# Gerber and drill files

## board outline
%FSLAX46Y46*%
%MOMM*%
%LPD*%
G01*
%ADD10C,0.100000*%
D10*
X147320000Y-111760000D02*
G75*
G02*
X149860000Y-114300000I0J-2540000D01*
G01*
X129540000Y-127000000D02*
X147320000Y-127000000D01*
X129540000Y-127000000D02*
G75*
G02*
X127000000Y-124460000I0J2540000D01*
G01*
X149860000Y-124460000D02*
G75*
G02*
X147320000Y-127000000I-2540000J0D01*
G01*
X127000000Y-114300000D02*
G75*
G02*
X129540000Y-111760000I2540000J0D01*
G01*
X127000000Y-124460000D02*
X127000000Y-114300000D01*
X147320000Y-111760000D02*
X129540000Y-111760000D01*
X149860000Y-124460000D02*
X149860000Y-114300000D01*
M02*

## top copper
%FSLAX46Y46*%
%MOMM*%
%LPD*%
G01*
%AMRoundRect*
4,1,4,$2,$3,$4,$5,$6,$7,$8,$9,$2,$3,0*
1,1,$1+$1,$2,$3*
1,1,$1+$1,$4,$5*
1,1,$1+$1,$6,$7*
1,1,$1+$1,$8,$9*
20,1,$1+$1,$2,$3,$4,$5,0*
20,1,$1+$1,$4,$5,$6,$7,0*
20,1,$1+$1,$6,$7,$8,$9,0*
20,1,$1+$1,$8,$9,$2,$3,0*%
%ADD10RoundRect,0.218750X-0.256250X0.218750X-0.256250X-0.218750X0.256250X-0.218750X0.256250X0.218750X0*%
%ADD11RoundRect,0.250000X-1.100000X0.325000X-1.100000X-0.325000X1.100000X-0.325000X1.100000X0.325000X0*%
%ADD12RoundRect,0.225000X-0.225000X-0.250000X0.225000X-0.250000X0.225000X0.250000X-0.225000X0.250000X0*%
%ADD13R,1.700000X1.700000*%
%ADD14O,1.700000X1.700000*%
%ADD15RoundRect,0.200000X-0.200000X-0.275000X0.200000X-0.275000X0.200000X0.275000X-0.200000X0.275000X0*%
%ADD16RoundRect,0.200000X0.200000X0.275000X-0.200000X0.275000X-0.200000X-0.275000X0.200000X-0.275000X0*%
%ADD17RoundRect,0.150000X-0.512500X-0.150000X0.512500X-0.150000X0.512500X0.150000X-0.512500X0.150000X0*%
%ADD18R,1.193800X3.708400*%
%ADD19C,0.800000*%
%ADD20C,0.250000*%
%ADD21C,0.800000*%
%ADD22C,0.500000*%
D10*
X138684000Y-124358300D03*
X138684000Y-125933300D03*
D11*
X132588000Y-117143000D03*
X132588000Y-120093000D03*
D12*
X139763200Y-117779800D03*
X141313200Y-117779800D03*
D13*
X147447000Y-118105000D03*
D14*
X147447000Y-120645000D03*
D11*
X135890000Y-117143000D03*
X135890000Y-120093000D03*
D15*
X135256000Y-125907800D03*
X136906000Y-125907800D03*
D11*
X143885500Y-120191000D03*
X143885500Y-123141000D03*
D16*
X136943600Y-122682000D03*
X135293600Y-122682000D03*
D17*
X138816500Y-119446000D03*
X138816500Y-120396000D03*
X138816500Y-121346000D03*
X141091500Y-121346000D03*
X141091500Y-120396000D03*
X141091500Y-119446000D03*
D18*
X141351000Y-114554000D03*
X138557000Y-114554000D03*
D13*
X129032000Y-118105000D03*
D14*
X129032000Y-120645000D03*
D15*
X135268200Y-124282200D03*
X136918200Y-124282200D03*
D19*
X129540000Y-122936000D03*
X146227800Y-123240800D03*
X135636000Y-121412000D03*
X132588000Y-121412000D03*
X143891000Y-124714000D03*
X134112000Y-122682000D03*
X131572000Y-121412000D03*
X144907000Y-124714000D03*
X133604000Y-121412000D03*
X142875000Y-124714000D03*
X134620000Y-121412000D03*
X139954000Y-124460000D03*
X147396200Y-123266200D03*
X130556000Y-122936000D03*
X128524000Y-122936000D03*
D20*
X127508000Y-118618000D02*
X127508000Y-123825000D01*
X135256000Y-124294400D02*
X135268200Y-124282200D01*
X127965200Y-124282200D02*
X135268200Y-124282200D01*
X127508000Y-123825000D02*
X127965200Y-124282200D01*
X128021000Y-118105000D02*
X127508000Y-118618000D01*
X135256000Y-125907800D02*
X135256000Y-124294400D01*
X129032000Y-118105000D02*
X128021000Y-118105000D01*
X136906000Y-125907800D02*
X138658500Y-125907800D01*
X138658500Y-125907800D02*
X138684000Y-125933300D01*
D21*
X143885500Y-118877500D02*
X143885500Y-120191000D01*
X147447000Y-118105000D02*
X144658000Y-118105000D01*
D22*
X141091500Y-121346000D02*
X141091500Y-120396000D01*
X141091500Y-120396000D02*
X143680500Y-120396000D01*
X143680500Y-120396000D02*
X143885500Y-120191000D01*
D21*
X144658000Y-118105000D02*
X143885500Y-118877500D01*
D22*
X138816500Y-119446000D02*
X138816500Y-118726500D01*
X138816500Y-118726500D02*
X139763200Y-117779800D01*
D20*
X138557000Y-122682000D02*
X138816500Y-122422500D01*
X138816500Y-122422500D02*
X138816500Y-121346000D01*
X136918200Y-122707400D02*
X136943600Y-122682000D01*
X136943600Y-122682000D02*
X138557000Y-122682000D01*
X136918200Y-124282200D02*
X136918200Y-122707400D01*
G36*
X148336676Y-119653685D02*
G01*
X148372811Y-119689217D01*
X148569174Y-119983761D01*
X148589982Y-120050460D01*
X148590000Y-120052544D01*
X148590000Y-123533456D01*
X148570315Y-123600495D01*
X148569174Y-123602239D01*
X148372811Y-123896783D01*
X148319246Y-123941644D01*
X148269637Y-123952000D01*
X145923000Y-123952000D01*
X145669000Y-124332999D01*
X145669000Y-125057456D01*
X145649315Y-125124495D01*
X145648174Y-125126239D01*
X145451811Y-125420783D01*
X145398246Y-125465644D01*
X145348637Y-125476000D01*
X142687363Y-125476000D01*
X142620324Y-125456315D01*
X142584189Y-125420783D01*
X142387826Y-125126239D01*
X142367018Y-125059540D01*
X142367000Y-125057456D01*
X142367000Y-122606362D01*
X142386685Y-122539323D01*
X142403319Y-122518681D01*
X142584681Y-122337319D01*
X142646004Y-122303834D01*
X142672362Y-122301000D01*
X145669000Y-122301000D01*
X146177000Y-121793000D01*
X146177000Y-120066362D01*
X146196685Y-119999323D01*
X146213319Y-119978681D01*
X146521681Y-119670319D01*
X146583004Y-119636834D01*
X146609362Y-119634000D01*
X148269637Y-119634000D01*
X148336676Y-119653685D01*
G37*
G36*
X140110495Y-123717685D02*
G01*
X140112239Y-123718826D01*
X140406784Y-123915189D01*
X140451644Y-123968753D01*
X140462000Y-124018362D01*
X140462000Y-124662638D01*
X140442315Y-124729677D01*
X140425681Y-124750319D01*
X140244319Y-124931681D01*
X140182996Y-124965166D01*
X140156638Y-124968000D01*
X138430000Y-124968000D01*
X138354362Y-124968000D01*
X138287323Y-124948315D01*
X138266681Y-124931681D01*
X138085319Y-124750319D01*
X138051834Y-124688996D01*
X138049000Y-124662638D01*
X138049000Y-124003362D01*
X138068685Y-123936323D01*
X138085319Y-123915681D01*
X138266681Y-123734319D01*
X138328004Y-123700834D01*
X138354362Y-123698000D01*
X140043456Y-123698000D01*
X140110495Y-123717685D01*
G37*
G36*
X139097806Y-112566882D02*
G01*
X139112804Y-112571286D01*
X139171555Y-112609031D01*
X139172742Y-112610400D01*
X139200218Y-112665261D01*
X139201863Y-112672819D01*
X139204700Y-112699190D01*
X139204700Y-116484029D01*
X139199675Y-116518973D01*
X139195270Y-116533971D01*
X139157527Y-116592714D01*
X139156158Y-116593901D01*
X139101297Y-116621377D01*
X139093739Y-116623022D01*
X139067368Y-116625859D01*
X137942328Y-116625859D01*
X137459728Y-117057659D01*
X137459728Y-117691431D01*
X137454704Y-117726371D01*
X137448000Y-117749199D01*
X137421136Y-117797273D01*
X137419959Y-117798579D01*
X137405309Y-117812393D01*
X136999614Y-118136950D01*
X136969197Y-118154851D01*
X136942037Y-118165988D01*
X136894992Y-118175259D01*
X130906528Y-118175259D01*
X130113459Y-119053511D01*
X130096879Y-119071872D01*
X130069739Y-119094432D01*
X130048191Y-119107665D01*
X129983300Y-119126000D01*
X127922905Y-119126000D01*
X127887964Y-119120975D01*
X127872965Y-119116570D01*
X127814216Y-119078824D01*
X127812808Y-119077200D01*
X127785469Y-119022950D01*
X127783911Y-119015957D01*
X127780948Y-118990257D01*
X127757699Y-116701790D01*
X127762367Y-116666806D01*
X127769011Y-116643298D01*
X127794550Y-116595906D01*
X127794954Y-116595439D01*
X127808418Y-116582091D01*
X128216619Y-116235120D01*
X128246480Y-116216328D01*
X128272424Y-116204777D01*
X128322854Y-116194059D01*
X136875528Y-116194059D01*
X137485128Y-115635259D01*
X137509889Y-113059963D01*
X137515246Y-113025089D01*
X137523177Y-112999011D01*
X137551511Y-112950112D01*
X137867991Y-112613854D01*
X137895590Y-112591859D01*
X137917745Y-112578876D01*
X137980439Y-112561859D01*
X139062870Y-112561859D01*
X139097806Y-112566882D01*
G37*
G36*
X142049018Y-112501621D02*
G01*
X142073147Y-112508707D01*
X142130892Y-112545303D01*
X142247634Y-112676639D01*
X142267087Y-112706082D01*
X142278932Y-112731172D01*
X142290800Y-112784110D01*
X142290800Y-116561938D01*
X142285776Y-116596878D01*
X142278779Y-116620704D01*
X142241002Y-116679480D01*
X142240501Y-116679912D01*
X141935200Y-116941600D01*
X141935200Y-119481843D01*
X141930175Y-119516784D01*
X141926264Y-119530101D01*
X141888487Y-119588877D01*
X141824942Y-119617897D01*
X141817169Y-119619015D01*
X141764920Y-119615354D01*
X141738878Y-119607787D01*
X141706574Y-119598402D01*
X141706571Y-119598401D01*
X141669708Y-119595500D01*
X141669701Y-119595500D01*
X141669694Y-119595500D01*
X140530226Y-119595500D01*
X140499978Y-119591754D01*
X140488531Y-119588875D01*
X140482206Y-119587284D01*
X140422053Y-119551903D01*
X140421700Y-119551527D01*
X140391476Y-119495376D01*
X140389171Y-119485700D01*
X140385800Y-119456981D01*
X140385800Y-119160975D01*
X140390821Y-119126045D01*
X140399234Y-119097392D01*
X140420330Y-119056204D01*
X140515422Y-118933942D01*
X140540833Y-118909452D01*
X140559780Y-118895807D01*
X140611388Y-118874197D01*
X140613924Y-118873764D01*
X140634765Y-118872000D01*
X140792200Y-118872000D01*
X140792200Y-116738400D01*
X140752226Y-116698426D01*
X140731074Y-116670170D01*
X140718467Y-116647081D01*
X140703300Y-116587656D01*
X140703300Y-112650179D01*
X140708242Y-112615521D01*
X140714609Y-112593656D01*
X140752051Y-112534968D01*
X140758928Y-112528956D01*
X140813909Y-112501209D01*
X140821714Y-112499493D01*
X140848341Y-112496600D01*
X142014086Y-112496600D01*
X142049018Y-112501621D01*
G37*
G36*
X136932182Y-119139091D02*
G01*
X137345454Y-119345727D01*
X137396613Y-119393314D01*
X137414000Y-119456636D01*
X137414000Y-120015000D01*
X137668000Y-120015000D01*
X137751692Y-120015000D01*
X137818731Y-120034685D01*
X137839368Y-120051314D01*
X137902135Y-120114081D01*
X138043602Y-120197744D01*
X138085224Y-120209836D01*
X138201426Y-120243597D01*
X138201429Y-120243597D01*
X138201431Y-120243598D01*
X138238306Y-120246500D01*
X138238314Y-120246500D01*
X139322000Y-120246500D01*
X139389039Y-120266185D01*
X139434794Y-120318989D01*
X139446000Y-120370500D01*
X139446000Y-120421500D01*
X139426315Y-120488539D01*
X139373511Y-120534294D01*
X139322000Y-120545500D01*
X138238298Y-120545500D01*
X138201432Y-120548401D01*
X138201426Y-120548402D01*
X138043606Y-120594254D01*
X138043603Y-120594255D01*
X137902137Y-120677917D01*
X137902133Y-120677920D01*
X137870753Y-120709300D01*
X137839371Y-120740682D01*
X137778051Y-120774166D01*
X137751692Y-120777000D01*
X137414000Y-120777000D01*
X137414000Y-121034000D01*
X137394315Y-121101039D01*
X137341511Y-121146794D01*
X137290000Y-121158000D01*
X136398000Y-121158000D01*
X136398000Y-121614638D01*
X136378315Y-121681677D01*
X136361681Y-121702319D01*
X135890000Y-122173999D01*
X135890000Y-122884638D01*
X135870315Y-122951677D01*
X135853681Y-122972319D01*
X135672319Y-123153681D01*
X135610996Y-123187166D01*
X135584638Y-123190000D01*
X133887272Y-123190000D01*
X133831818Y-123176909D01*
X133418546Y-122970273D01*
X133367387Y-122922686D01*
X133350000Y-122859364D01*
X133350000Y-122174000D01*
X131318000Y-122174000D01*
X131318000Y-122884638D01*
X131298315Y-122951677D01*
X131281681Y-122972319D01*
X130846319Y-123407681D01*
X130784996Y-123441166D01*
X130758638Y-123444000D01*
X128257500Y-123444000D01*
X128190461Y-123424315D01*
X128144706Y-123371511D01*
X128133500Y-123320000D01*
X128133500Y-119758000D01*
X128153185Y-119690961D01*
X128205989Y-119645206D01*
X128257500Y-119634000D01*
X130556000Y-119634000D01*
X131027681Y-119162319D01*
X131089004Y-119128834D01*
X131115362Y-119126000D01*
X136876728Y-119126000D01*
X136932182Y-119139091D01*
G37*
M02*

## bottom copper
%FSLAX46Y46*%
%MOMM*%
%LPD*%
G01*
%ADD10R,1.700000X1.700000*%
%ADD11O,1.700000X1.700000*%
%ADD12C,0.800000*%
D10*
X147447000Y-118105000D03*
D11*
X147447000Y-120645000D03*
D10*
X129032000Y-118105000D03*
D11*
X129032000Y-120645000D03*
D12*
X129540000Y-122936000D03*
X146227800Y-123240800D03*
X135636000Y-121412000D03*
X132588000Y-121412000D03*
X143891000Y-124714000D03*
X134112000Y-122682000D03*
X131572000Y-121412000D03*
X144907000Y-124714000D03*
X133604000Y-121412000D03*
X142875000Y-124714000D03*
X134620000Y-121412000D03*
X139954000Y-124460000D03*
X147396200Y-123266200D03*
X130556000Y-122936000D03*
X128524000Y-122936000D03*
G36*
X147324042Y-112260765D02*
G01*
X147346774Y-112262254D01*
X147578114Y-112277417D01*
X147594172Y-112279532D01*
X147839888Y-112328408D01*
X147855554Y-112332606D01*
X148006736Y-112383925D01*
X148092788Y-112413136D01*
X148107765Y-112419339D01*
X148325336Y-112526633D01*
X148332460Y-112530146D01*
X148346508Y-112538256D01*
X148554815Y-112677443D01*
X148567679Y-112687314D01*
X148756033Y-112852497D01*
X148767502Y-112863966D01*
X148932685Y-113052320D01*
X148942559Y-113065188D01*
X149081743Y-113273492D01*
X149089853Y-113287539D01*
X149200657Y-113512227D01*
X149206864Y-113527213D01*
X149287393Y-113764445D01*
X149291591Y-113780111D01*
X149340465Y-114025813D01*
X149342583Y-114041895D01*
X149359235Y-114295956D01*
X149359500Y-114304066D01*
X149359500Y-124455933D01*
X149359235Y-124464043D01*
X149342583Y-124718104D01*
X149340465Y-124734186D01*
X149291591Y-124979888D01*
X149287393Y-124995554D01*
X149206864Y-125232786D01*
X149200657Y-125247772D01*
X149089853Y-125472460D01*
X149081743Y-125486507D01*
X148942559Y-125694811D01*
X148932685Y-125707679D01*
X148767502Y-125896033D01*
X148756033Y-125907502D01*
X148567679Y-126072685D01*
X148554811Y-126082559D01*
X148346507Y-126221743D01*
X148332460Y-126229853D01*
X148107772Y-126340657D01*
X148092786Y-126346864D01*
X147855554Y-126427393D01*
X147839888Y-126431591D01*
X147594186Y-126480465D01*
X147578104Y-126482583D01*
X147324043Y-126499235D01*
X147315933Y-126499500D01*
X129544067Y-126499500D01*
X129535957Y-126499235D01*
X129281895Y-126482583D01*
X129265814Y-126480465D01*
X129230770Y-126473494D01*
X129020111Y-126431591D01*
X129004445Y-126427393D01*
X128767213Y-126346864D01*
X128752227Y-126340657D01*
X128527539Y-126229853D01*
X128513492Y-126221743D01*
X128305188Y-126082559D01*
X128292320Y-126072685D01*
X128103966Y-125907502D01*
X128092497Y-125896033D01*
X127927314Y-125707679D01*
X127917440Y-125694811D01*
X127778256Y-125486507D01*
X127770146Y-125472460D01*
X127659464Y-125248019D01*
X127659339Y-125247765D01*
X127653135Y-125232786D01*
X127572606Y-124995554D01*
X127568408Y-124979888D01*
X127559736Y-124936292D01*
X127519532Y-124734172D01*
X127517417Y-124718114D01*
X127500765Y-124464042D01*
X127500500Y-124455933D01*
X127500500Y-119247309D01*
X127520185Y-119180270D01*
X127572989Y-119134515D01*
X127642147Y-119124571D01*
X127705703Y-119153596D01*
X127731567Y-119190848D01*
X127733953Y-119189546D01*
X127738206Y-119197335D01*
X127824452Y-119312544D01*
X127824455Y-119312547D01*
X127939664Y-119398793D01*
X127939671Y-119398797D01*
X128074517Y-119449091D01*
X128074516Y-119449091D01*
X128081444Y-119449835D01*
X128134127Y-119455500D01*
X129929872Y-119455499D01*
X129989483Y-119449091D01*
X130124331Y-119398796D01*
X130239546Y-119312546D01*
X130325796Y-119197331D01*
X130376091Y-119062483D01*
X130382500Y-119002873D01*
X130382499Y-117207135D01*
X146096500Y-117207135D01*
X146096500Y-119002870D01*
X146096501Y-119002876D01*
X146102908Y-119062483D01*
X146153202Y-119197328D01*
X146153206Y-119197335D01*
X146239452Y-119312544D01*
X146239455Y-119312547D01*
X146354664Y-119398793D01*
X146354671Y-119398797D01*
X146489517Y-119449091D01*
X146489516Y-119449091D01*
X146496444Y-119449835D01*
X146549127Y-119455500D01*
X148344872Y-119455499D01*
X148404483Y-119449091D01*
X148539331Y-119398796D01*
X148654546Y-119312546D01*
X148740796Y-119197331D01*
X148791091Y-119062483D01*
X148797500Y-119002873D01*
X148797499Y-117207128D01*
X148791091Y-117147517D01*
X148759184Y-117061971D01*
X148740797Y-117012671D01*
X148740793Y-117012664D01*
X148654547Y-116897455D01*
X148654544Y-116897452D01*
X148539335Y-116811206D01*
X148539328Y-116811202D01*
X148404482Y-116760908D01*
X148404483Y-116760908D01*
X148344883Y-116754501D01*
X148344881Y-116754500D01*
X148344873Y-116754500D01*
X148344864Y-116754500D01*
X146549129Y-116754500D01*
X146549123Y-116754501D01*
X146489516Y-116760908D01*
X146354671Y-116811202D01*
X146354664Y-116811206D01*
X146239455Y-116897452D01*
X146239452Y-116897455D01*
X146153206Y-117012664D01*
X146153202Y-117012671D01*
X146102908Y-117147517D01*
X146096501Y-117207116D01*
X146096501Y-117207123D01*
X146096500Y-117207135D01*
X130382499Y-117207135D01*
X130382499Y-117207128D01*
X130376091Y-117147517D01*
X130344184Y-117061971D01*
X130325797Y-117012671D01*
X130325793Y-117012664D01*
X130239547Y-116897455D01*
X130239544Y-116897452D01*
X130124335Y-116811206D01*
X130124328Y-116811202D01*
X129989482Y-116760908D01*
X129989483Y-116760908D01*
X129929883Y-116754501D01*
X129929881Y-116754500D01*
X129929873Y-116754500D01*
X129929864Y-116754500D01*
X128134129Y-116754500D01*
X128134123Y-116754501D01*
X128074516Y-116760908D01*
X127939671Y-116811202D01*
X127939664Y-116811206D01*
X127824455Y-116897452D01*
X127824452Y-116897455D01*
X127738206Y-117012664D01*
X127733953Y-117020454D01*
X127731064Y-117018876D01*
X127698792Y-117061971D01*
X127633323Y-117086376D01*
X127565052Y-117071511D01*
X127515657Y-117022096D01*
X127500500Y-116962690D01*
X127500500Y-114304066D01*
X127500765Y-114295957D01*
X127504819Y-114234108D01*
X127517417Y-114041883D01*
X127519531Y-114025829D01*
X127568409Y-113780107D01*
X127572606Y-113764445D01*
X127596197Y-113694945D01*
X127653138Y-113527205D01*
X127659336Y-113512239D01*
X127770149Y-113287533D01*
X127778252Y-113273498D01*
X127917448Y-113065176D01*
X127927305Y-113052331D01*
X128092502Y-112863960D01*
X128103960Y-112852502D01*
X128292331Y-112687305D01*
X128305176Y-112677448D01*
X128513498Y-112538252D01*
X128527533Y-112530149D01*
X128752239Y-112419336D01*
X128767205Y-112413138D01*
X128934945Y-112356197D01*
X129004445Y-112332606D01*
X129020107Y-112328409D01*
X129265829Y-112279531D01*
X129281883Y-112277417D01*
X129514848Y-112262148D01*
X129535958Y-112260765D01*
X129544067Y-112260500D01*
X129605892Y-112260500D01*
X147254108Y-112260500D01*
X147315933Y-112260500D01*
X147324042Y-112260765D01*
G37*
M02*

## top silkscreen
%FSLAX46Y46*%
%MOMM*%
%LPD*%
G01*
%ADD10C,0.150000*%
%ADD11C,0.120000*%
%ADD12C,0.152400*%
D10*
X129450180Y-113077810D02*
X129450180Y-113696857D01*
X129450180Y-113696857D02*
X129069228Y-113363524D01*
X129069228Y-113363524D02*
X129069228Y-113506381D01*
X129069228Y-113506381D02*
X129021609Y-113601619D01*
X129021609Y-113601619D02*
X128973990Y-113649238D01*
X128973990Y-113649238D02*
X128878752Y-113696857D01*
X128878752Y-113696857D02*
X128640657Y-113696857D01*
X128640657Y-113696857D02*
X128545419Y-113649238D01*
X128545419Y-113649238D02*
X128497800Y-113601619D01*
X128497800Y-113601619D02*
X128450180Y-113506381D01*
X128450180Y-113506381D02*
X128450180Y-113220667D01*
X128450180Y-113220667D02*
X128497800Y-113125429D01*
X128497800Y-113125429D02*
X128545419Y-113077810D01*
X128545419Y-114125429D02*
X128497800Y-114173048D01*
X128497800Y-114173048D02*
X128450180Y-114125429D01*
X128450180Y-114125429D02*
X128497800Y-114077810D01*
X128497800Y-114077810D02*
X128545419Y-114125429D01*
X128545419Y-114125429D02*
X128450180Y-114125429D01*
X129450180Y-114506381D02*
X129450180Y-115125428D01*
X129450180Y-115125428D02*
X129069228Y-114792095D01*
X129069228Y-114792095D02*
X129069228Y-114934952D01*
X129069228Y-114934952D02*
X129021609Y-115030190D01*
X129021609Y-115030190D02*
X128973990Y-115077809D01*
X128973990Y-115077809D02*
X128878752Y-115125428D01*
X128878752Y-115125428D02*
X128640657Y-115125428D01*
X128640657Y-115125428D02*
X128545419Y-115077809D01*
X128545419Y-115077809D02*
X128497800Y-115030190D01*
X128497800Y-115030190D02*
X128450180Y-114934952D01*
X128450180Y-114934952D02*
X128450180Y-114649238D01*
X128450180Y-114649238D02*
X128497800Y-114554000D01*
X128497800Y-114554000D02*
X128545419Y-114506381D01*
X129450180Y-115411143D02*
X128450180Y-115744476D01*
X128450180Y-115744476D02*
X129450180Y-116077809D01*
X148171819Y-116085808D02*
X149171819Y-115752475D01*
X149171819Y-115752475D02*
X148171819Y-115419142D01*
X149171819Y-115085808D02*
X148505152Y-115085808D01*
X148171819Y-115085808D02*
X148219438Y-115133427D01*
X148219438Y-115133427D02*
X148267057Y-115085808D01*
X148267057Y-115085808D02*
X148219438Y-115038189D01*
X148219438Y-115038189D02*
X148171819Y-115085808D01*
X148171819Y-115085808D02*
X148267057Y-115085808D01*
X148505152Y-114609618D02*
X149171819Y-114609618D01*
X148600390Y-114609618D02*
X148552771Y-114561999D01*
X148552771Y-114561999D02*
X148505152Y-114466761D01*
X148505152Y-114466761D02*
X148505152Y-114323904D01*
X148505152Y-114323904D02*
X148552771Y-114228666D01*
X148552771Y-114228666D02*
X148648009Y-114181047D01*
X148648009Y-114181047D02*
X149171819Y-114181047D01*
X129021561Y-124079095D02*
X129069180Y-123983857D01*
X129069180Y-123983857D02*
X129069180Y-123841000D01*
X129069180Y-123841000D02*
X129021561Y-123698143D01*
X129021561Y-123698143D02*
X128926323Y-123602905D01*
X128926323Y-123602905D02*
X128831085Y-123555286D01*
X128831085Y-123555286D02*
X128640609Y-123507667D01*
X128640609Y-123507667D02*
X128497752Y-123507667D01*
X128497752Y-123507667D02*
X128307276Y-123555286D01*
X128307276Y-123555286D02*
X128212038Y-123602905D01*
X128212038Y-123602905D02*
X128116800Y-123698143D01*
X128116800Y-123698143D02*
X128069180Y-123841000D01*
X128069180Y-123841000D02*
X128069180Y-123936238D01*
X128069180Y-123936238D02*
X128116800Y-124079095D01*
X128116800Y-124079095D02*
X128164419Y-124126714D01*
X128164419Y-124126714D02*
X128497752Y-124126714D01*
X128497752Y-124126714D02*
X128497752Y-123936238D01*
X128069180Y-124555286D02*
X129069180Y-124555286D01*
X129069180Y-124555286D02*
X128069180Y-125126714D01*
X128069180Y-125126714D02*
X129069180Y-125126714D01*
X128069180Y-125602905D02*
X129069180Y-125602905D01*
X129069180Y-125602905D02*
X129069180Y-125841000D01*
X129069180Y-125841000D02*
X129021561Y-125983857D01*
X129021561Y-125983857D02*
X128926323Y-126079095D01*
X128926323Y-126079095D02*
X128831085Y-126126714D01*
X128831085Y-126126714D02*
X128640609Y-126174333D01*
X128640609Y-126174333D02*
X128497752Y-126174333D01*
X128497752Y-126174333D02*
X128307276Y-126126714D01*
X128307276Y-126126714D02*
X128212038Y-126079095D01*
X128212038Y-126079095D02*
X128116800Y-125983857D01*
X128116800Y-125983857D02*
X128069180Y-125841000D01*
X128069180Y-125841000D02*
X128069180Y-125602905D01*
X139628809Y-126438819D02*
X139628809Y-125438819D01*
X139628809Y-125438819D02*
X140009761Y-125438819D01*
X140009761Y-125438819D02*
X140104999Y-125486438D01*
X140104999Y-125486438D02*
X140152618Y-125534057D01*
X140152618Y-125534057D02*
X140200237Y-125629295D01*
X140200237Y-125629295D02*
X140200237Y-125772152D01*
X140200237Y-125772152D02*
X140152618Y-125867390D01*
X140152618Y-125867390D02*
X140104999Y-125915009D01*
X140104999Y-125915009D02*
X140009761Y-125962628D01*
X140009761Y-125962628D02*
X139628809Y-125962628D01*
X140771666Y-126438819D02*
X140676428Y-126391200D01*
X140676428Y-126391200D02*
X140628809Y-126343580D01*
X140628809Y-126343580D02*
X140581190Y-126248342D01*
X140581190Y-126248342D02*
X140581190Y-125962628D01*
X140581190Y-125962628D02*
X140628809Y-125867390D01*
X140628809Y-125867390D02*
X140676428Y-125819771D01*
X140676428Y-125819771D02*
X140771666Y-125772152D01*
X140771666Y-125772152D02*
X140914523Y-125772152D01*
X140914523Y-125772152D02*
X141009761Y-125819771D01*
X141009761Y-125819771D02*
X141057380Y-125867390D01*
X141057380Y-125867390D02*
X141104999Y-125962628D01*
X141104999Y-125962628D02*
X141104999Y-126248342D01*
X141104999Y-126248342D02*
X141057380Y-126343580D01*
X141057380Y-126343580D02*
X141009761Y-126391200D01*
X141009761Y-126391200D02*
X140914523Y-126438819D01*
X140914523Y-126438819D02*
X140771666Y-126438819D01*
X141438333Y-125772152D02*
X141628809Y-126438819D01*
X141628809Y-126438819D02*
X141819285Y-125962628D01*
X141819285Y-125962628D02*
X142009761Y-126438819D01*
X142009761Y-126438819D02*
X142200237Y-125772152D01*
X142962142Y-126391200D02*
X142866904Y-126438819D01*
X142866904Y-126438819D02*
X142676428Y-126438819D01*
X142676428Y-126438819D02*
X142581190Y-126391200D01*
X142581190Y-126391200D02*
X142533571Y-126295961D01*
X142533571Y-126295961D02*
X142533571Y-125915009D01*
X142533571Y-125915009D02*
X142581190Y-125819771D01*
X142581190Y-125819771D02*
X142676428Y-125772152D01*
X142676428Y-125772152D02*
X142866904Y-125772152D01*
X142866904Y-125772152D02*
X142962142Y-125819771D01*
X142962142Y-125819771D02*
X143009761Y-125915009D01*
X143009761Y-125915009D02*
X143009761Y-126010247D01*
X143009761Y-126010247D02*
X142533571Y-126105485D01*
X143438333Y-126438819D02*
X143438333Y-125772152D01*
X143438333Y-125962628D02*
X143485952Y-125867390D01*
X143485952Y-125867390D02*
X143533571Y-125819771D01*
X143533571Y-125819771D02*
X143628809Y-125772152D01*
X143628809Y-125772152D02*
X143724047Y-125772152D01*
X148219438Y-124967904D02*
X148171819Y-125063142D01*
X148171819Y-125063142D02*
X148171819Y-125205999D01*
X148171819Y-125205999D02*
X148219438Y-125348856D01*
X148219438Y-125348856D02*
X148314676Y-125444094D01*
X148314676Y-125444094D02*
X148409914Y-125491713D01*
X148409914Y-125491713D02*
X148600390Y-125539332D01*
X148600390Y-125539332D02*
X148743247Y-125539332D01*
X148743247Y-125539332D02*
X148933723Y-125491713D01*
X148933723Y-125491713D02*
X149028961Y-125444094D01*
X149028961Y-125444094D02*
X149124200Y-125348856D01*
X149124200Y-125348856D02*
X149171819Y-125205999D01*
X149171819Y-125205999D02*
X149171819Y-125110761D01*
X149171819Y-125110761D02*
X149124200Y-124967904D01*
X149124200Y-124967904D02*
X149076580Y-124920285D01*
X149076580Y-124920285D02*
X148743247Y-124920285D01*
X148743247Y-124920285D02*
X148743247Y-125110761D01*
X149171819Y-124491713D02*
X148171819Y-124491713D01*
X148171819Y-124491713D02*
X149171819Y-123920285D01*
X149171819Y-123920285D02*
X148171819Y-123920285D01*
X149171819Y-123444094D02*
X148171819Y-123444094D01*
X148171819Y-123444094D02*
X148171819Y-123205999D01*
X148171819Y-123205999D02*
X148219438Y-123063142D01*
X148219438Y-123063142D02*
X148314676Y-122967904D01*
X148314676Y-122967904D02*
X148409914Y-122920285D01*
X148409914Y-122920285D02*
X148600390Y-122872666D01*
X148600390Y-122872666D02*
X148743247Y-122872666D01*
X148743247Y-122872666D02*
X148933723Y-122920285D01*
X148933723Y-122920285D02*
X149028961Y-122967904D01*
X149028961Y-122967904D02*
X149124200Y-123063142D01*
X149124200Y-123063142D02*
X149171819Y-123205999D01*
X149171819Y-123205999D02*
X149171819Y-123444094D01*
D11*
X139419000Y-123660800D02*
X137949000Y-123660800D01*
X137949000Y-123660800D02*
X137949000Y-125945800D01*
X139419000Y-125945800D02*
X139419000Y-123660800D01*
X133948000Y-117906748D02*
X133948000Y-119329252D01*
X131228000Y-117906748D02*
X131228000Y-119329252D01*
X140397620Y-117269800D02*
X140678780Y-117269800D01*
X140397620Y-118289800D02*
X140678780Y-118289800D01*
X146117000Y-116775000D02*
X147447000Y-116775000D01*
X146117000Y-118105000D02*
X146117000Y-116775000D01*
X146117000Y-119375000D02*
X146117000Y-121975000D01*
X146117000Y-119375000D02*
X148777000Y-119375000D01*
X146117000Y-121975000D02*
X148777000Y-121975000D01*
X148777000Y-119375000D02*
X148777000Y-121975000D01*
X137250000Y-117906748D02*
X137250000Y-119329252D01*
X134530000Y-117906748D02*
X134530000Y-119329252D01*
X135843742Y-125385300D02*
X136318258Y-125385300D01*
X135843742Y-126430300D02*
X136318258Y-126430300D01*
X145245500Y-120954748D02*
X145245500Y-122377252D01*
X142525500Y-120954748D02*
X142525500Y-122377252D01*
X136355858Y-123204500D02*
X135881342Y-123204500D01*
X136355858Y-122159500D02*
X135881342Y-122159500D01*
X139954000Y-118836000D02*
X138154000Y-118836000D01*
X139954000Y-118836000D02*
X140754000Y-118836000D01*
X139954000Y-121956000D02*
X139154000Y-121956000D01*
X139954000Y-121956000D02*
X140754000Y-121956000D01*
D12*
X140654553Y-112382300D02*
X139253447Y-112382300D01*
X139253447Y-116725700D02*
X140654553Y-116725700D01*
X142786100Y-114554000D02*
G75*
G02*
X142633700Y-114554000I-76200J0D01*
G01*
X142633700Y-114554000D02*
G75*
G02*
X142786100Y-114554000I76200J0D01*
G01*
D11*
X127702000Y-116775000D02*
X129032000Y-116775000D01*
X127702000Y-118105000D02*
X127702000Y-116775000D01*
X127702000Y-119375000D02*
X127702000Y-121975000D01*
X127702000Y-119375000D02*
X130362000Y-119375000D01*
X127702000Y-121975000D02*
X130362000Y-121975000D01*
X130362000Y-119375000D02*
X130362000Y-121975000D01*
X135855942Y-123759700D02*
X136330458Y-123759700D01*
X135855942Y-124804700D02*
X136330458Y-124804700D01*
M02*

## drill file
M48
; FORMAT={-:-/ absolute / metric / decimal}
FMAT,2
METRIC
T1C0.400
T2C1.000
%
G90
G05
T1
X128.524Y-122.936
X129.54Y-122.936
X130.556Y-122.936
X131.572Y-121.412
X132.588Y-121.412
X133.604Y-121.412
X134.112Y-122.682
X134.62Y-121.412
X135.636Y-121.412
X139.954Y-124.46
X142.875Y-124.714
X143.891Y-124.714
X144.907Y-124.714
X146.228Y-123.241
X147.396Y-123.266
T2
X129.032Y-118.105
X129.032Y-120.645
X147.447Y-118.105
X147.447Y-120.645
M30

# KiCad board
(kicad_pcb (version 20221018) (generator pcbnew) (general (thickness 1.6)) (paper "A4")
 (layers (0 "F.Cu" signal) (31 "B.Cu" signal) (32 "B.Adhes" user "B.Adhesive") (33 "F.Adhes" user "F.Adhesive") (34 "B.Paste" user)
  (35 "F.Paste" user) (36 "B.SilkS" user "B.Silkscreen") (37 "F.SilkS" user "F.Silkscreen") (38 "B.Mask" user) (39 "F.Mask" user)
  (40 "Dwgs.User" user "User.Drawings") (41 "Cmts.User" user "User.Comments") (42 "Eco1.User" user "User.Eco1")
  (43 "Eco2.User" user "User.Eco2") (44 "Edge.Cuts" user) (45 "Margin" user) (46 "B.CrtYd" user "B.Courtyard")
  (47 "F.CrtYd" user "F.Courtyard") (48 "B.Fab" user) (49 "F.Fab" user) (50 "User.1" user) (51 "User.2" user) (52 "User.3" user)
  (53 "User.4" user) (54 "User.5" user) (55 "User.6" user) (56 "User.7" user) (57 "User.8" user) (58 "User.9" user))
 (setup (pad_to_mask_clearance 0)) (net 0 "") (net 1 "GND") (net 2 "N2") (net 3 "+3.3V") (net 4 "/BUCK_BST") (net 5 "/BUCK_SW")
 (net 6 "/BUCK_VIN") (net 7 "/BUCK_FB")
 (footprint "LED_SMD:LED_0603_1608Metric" (layer "F.Cu") (at 138.684 125.1458 -90)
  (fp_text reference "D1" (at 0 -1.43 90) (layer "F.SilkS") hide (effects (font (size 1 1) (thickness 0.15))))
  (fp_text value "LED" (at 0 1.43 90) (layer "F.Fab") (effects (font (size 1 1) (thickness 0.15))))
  (fp_line (start -1.485 -0.735) (end -1.485 0.735) (stroke (width 0.12) (type solid)) (layer "F.SilkS"))
  (fp_line (start -1.485 0.735) (end 0.8 0.735) (stroke (width 0.12) (type solid)) (layer "F.SilkS"))
  (fp_line (start 0.8 -0.735) (end -1.485 -0.735) (stroke (width 0.12) (type solid)) (layer "F.SilkS"))
  (pad "1" smd roundrect (at -0.7875 0 270) (size 0.875 0.95) (layers "F.Cu" "F.Paste" "F.Mask") (roundrect_rratio 0.25) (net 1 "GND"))
  (pad "2" smd roundrect (at 0.7875 0 270) (size 0.875 0.95) (layers "F.Cu" "F.Paste" "F.Mask") (roundrect_rratio 0.25) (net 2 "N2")))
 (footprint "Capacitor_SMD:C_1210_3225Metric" (layer "F.Cu") (at 132.588 118.618 -90)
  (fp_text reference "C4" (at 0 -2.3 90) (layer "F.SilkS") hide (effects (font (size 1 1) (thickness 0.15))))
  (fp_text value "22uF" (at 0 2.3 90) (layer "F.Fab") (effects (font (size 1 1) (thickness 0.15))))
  (fp_line (start -0.711252 -1.36) (end 0.711252 -1.36) (stroke (width 0.12) (type solid)) (layer "F.SilkS"))
  (fp_line (start -0.711252 1.36) (end 0.711252 1.36) (stroke (width 0.12) (type solid)) (layer "F.SilkS"))
  (pad "1" smd roundrect (at -1.475 0 270) (size 1.15 2.7) (layers "F.Cu" "F.Paste" "F.Mask") (roundrect_rratio 0.217391) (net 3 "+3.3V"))
  (pad "2" smd roundrect (at 1.475 0 270) (size 1.15 2.7) (layers "F.Cu" "F.Paste" "F.Mask") (roundrect_rratio 0.217391) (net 1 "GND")))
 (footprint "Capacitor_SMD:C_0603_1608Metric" (layer "F.Cu") (at 140.5382 117.7798)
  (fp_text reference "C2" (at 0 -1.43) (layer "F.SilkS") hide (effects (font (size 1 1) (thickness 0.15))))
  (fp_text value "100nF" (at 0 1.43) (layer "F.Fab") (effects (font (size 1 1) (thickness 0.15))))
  (fp_line (start -0.14058 -0.51) (end 0.14058 -0.51) (stroke (width 0.12) (type solid)) (layer "F.SilkS"))
  (fp_line (start -0.14058 0.51) (end 0.14058 0.51) (stroke (width 0.12) (type solid)) (layer "F.SilkS"))
  (pad "1" smd roundrect (at -0.775 0) (size 0.9 0.95) (layers "F.Cu" "F.Paste" "F.Mask") (roundrect_rratio 0.25) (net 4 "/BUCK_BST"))
  (pad "2" smd roundrect (at 0.775 0) (size 0.9 0.95) (layers "F.Cu" "F.Paste" "F.Mask") (roundrect_rratio 0.25) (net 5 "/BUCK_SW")))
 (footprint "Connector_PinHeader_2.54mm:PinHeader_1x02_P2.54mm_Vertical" (layer "F.Cu") (at 147.447 118.105)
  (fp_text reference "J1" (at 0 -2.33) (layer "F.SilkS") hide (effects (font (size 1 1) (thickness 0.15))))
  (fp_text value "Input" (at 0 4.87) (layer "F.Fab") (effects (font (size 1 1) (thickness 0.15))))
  (fp_line (start -1.33 -1.33) (end 0 -1.33) (stroke (width 0.12) (type solid)) (layer "F.SilkS"))
  (fp_line (start -1.33 0) (end -1.33 -1.33) (stroke (width 0.12) (type solid)) (layer "F.SilkS"))
  (fp_line (start -1.33 1.27) (end -1.33 3.87) (stroke (width 0.12) (type solid)) (layer "F.SilkS"))
  (fp_line (start -1.33 1.27) (end 1.33 1.27) (stroke (width 0.12) (type solid)) (layer "F.SilkS"))
  (fp_line (start -1.33 3.87) (end 1.33 3.87) (stroke (width 0.12) (type solid)) (layer "F.SilkS"))
  (fp_line (start 1.33 1.27) (end 1.33 3.87) (stroke (width 0.12) (type solid)) (layer "F.SilkS"))
  (pad "1" thru_hole rect (at 0 0) (size 1.7 1.7) (drill 1) (layers "*.Cu" "*.Mask") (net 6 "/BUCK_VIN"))
  (pad "2" thru_hole oval (at 0 2.54) (size 1.7 1.7) (drill 1) (layers "*.Cu" "*.Mask") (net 1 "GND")))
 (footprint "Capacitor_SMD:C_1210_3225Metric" (layer "F.Cu") (at 135.89 118.618 -90)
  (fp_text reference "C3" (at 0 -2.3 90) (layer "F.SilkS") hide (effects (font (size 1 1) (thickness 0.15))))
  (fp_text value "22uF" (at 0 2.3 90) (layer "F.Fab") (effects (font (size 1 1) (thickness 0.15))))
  (fp_line (start -0.711252 -1.36) (end 0.711252 -1.36) (stroke (width 0.12) (type solid)) (layer "F.SilkS"))
  (fp_line (start -0.711252 1.36) (end 0.711252 1.36) (stroke (width 0.12) (type solid)) (layer "F.SilkS"))
  (pad "1" smd roundrect (at -1.475 0 270) (size 1.15 2.7) (layers "F.Cu" "F.Paste" "F.Mask") (roundrect_rratio 0.217391) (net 3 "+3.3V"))
  (pad "2" smd roundrect (at 1.475 0 270) (size 1.15 2.7) (layers "F.Cu" "F.Paste" "F.Mask") (roundrect_rratio 0.217391) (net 1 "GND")))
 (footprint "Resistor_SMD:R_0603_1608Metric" (layer "F.Cu") (at 136.081 125.9078)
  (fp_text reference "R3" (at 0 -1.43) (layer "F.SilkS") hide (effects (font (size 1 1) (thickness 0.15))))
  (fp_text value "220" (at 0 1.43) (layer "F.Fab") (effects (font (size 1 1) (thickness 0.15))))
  (fp_line (start -0.237258 -0.5225) (end 0.237258 -0.5225) (stroke (width 0.12) (type solid)) (layer "F.SilkS"))
  (fp_line (start -0.237258 0.5225) (end 0.237258 0.5225) (stroke (width 0.12) (type solid)) (layer "F.SilkS"))
  (pad "1" smd roundrect (at -0.825 0) (size 0.8 0.95) (layers "F.Cu" "F.Paste" "F.Mask") (roundrect_rratio 0.25) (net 3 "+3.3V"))
  (pad "2" smd roundrect (at 0.825 0) (size 0.8 0.95) (layers "F.Cu" "F.Paste" "F.Mask") (roundrect_rratio 0.25) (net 2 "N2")))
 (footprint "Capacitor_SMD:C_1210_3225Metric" (layer "F.Cu") (at 143.8855 121.666 -90)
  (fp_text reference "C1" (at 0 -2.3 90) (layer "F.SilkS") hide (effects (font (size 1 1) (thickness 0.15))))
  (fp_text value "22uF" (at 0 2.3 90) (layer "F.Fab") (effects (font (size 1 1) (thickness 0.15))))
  (fp_line (start -0.711252 -1.36) (end 0.711252 -1.36) (stroke (width 0.12) (type solid)) (layer "F.SilkS"))
  (fp_line (start -0.711252 1.36) (end 0.711252 1.36) (stroke (width 0.12) (type solid)) (layer "F.SilkS"))
  (pad "1" smd roundrect (at -1.475 0 270) (size 1.15 2.7) (layers "F.Cu" "F.Paste" "F.Mask") (roundrect_rratio 0.217391)
   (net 6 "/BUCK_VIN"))
  (pad "2" smd roundrect (at 1.475 0 270) (size 1.15 2.7) (layers "F.Cu" "F.Paste" "F.Mask") (roundrect_rratio 0.217391) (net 1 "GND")))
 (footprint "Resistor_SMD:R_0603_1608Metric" (layer "F.Cu") (at 136.1186 122.682 180)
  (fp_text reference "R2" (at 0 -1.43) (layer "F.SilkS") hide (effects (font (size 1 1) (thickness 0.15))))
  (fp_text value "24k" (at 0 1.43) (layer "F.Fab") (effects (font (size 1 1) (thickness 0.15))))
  (fp_line (start -0.237258 -0.5225) (end 0.237258 -0.5225) (stroke (width 0.12) (type solid)) (layer "F.SilkS"))
  (fp_line (start -0.237258 0.5225) (end 0.237258 0.5225) (stroke (width 0.12) (type solid)) (layer "F.SilkS"))
  (pad "1" smd roundrect (at -0.825 0 180) (size 0.8 0.95) (layers "F.Cu" "F.Paste" "F.Mask") (roundrect_rratio 0.25) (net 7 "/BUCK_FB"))
  (pad "2" smd roundrect (at 0.825 0 180) (size 0.8 0.95) (layers "F.Cu" "F.Paste" "F.Mask") (roundrect_rratio 0.25) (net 1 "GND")))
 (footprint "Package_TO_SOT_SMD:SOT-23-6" (layer "F.Cu") (at 139.954 120.396)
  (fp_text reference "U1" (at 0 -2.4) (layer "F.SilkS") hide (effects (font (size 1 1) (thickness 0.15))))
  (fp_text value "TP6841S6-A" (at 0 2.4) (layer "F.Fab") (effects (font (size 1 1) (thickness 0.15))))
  (fp_line (start 0 -1.56) (end -1.8 -1.56) (stroke (width 0.12) (type solid)) (layer "F.SilkS"))
  (fp_line (start 0 -1.56) (end 0.8 -1.56) (stroke (width 0.12) (type solid)) (layer "F.SilkS"))
  (fp_line (start 0 1.56) (end -0.8 1.56) (stroke (width 0.12) (type solid)) (layer "F.SilkS"))
  (fp_line (start 0 1.56) (end 0.8 1.56) (stroke (width 0.12) (type solid)) (layer "F.SilkS"))
  (pad "1" smd roundrect (at -1.1375 -0.95) (size 1.325 0.6) (layers "F.Cu" "F.Paste" "F.Mask") (roundrect_rratio 0.25) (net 4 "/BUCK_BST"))
  (pad "2" smd roundrect (at -1.1375 0) (size 1.325 0.6) (layers "F.Cu" "F.Paste" "F.Mask") (roundrect_rratio 0.25) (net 1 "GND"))
  (pad "3" smd roundrect (at -1.1375 0.95) (size 1.325 0.6) (layers "F.Cu" "F.Paste" "F.Mask") (roundrect_rratio 0.25) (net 7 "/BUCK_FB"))
  (pad "4" smd roundrect (at 1.1375 0.95) (size 1.325 0.6) (layers "F.Cu" "F.Paste" "F.Mask") (roundrect_rratio 0.25) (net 6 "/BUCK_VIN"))
  (pad "5" smd roundrect (at 1.1375 0) (size 1.325 0.6) (layers "F.Cu" "F.Paste" "F.Mask") (roundrect_rratio 0.25) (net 6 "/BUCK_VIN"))
  (pad "6" smd roundrect (at 1.1375 -0.95) (size 1.325 0.6) (layers "F.Cu" "F.Paste" "F.Mask") (roundrect_rratio 0.25) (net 5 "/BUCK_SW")))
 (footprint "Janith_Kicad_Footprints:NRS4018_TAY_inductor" (layer "F.Cu") (at 139.954 114.554 180)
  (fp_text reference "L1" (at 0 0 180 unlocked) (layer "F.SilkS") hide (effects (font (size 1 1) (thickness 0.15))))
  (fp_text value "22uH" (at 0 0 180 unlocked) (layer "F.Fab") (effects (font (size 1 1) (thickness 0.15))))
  (fp_line (start -0.700553 2.1717) (end 0.700553 2.1717) (stroke (width 0.1524) (type solid)) (layer "F.SilkS"))
  (fp_line (start 0.700553 -2.1717) (end -0.700553 -2.1717) (stroke (width 0.1524) (type solid)) (layer "F.SilkS"))
  (fp_circle (center -2.7559 0) (end -2.6797 0) (stroke (width 0.1524) (type solid)) (fill none) (layer "F.SilkS"))
  (pad "1" smd rect (at -1.397 0 180) (size 1.1938 3.7084) (layers "F.Cu" "F.Paste" "F.Mask") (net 5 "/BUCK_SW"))
  (pad "2" smd rect (at 1.397 0 180) (size 1.1938 3.7084) (layers "F.Cu" "F.Paste" "F.Mask") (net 3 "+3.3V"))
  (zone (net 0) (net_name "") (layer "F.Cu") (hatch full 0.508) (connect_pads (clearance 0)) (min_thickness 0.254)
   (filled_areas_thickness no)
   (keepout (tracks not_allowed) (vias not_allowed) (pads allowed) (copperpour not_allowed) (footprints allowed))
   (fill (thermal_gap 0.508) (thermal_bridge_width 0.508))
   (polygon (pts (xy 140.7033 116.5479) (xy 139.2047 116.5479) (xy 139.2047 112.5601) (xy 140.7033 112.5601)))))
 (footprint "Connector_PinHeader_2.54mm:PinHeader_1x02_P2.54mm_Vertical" (layer "F.Cu") (at 129.032 118.105)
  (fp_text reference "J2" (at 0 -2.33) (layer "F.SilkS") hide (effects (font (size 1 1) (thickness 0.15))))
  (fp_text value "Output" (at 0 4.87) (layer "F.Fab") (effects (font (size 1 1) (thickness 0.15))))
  (fp_line (start -1.33 -1.33) (end 0 -1.33) (stroke (width 0.12) (type solid)) (layer "F.SilkS"))
  (fp_line (start -1.33 0) (end -1.33 -1.33) (stroke (width 0.12) (type solid)) (layer "F.SilkS"))
  (fp_line (start -1.33 1.27) (end -1.33 3.87) (stroke (width 0.12) (type solid)) (layer "F.SilkS"))
  (fp_line (start -1.33 1.27) (end 1.33 1.27) (stroke (width 0.12) (type solid)) (layer "F.SilkS"))
  (fp_line (start -1.33 3.87) (end 1.33 3.87) (stroke (width 0.12) (type solid)) (layer "F.SilkS"))
  (fp_line (start 1.33 1.27) (end 1.33 3.87) (stroke (width 0.12) (type solid)) (layer "F.SilkS"))
  (pad "1" thru_hole rect (at 0 0) (size 1.7 1.7) (drill 1) (layers "*.Cu" "*.Mask") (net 3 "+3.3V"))
  (pad "2" thru_hole oval (at 0 2.54) (size 1.7 1.7) (drill 1) (layers "*.Cu" "*.Mask") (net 1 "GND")))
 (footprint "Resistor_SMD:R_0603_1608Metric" (layer "F.Cu") (at 136.0932 124.2822)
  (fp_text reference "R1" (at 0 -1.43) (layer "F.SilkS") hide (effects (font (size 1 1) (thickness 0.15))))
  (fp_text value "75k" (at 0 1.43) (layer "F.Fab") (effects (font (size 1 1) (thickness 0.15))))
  (fp_line (start -0.237258 -0.5225) (end 0.237258 -0.5225) (stroke (width 0.12) (type solid)) (layer "F.SilkS"))
  (fp_line (start -0.237258 0.5225) (end 0.237258 0.5225) (stroke (width 0.12) (type solid)) (layer "F.SilkS"))
  (pad "1" smd roundrect (at -0.825 0) (size 0.8 0.95) (layers "F.Cu" "F.Paste" "F.Mask") (roundrect_rratio 0.25) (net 3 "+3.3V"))
  (pad "2" smd roundrect (at 0.825 0) (size 0.8 0.95) (layers "F.Cu" "F.Paste" "F.Mask") (roundrect_rratio 0.25) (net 7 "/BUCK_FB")))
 (gr_arc (start 147.32 111.76) (mid 149.116051 112.503949) (end 149.86 114.3) (stroke (width 0.1) (type default)) (layer "Edge.Cuts"))
 (gr_line (start 129.54 127) (end 147.32 127) (stroke (width 0.1) (type default)) (layer "Edge.Cuts"))
 (gr_arc (start 129.54 127) (mid 127.743949 126.256051) (end 127 124.46) (stroke (width 0.1) (type default)) (layer "Edge.Cuts"))
 (gr_arc (start 149.86 124.46) (mid 149.116051 126.256051) (end 147.32 127) (stroke (width 0.1) (type default)) (layer "Edge.Cuts"))
 (gr_arc (start 127 114.3) (mid 127.743949 112.503949) (end 129.54 111.76) (stroke (width 0.1) (type default)) (layer "Edge.Cuts"))
 (gr_line (start 127 124.46) (end 127 114.3) (stroke (width 0.1) (type default)) (layer "Edge.Cuts"))
 (gr_line (start 147.32 111.76) (end 129.54 111.76) (stroke (width 0.1) (type default)) (layer "Edge.Cuts"))
 (gr_line (start 149.86 124.46) (end 149.86 114.3) (stroke (width 0.1) (type default)) (layer "Edge.Cuts"))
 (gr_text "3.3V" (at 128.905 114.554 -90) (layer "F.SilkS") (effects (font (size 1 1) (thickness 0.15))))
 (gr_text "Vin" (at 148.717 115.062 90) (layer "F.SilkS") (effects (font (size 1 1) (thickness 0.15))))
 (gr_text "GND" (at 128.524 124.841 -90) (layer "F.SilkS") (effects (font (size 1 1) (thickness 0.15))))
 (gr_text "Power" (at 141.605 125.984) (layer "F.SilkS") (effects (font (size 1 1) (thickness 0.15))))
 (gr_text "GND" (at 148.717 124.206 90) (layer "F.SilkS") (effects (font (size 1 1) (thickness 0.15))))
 (via (at 129.54 122.936) (size 0.8) (drill 0.4) (layers "F.Cu" "B.Cu") (free) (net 1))
 (via (at 146.2278 123.2408) (size 0.8) (drill 0.4) (layers "F.Cu" "B.Cu") (free) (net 1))
 (via (at 135.636 121.412) (size 0.8) (drill 0.4) (layers "F.Cu" "B.Cu") (free) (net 1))
 (via (at 132.588 121.412) (size 0.8) (drill 0.4) (layers "F.Cu" "B.Cu") (free) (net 1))
 (via (at 143.891 124.714) (size 0.8) (drill 0.4) (layers "F.Cu" "B.Cu") (free) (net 1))
 (via (at 134.112 122.682) (size 0.8) (drill 0.4) (layers "F.Cu" "B.Cu") (free) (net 1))
 (via (at 131.572 121.412) (size 0.8) (drill 0.4) (layers "F.Cu" "B.Cu") (free) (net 1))
 (via (at 144.907 124.714) (size 0.8) (drill 0.4) (layers "F.Cu" "B.Cu") (free) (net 1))
 (via (at 133.604 121.412) (size 0.8) (drill 0.4) (layers "F.Cu" "B.Cu") (free) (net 1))
 (via (at 142.875 124.714) (size 0.8) (drill 0.4) (layers "F.Cu" "B.Cu") (free) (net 1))
 (via (at 134.62 121.412) (size 0.8) (drill 0.4) (layers "F.Cu" "B.Cu") (free) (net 1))
 (via (at 139.954 124.46) (size 0.8) (drill 0.4) (layers "F.Cu" "B.Cu") (free) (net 1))
 (via (at 147.3962 123.2662) (size 0.8) (drill 0.4) (layers "F.Cu" "B.Cu") (free) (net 1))
 (via (at 130.556 122.936) (size 0.8) (drill 0.4) (layers "F.Cu" "B.Cu") (free) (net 1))
 (via (at 128.524 122.936) (size 0.8) (drill 0.4) (layers "F.Cu" "B.Cu") (free) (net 1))
 (segment (start 127.508 118.618) (end 127.508 123.825) (width 0.25) (layer "F.Cu") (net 3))
 (segment (start 135.256 124.2944) (end 135.2682 124.2822) (width 0.25) (layer "F.Cu") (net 3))
 (segment (start 127.9652 124.2822) (end 135.2682 124.2822) (width 0.25) (layer "F.Cu") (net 3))
 (segment (start 127.508 123.825) (end 127.9652 124.2822) (width 0.25) (layer "F.Cu") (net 3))
 (segment (start 128.021 118.105) (end 127.508 118.618) (width 0.25) (layer "F.Cu") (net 3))
 (segment (start 135.256 125.9078) (end 135.256 124.2944) (width 0.25) (layer "F.Cu") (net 3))
 (segment (start 129.032 118.105) (end 128.021 118.105) (width 0.25) (layer "F.Cu") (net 3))
 (segment (start 136.906 125.9078) (end 138.6585 125.9078) (width 0.25) (layer "F.Cu") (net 2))
 (segment (start 138.6585 125.9078) (end 138.684 125.9333) (width 0.25) (layer "F.Cu") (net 2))
 (segment (start 143.8855 118.8775) (end 143.8855 120.191) (width 0.8) (layer "F.Cu") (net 6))
 (segment (start 147.447 118.105) (end 144.658 118.105) (width 0.8) (layer "F.Cu") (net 6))
 (segment (start 141.0915 121.346) (end 141.0915 120.396) (width 0.5) (layer "F.Cu") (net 6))
 (segment (start 141.0915 120.396) (end 143.6805 120.396) (width 0.5) (layer "F.Cu") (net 6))
 (segment (start 143.6805 120.396) (end 143.8855 120.191) (width 0.5) (layer "F.Cu") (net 6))
 (segment (start 144.658 118.105) (end 143.8855 118.8775) (width 0.8) (layer "F.Cu") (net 6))
 (segment (start 138.8165 119.446) (end 138.8165 118.7265) (width 0.5) (layer "F.Cu") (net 4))
 (segment (start 138.8165 118.7265) (end 139.7632 117.7798) (width 0.5) (layer "F.Cu") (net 4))
 (segment (start 138.557 122.682) (end 138.8165 122.4225) (width 0.25) (layer "F.Cu") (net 7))
 (segment (start 138.8165 122.4225) (end 138.8165 121.346) (width 0.25) (layer "F.Cu") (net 7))
 (segment (start 136.9182 122.7074) (end 136.9436 122.682) (width 0.25) (layer "F.Cu") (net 7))
 (segment (start 136.9436 122.682) (end 138.557 122.682) (width 0.25) (layer "F.Cu") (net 7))
 (segment (start 136.9182 124.2822) (end 136.9182 122.7074) (width 0.25) (layer "F.Cu") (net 7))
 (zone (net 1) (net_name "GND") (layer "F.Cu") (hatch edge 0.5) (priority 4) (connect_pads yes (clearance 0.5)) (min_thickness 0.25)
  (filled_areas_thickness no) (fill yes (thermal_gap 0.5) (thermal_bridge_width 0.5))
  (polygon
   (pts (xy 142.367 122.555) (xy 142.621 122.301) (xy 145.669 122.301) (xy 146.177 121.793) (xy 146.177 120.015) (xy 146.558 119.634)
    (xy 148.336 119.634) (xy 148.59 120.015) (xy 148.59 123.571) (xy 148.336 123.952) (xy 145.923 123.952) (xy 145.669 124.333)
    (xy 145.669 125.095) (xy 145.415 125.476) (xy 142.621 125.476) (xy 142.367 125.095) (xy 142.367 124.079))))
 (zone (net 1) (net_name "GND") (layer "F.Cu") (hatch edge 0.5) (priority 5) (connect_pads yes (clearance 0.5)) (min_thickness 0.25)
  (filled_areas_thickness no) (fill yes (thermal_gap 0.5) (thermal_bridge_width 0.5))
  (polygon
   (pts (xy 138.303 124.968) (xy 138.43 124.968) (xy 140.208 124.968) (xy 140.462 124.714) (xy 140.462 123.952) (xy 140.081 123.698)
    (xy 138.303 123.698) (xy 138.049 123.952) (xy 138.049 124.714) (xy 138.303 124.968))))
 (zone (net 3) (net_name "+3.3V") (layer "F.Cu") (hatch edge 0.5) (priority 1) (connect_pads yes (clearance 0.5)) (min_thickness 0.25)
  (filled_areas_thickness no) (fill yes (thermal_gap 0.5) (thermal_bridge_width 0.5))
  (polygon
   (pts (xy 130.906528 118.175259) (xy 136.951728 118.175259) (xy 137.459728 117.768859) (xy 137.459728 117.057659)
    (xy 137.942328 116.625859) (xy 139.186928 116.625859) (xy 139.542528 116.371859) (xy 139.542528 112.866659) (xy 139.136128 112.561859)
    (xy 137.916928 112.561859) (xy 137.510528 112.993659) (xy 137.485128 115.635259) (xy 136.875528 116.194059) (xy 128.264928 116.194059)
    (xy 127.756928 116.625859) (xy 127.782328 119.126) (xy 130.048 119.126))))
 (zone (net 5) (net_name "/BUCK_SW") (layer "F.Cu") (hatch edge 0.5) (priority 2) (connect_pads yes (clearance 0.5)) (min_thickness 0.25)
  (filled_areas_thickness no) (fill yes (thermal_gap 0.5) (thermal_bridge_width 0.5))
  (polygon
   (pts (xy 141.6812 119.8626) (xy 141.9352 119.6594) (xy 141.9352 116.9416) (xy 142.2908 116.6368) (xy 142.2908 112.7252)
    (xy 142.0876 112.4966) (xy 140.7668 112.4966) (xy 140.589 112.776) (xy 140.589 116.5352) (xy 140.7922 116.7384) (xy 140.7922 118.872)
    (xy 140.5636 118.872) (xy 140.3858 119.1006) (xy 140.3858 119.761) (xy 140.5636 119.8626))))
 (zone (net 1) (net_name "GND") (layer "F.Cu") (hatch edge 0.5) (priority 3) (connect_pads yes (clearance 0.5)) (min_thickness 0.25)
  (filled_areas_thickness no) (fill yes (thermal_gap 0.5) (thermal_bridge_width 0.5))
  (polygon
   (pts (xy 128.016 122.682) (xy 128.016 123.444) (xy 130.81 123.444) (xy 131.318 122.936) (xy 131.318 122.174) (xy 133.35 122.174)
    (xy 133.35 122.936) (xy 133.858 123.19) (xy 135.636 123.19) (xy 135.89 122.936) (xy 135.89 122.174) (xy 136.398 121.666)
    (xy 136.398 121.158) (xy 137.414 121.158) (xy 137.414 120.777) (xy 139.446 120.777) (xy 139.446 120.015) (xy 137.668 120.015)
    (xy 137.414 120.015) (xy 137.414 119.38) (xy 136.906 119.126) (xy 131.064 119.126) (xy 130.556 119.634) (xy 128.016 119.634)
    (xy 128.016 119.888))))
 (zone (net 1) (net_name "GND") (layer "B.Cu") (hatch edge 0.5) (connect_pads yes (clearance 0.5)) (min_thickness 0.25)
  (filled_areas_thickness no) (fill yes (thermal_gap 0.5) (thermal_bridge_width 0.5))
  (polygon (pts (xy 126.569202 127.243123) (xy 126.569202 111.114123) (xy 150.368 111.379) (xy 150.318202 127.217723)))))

